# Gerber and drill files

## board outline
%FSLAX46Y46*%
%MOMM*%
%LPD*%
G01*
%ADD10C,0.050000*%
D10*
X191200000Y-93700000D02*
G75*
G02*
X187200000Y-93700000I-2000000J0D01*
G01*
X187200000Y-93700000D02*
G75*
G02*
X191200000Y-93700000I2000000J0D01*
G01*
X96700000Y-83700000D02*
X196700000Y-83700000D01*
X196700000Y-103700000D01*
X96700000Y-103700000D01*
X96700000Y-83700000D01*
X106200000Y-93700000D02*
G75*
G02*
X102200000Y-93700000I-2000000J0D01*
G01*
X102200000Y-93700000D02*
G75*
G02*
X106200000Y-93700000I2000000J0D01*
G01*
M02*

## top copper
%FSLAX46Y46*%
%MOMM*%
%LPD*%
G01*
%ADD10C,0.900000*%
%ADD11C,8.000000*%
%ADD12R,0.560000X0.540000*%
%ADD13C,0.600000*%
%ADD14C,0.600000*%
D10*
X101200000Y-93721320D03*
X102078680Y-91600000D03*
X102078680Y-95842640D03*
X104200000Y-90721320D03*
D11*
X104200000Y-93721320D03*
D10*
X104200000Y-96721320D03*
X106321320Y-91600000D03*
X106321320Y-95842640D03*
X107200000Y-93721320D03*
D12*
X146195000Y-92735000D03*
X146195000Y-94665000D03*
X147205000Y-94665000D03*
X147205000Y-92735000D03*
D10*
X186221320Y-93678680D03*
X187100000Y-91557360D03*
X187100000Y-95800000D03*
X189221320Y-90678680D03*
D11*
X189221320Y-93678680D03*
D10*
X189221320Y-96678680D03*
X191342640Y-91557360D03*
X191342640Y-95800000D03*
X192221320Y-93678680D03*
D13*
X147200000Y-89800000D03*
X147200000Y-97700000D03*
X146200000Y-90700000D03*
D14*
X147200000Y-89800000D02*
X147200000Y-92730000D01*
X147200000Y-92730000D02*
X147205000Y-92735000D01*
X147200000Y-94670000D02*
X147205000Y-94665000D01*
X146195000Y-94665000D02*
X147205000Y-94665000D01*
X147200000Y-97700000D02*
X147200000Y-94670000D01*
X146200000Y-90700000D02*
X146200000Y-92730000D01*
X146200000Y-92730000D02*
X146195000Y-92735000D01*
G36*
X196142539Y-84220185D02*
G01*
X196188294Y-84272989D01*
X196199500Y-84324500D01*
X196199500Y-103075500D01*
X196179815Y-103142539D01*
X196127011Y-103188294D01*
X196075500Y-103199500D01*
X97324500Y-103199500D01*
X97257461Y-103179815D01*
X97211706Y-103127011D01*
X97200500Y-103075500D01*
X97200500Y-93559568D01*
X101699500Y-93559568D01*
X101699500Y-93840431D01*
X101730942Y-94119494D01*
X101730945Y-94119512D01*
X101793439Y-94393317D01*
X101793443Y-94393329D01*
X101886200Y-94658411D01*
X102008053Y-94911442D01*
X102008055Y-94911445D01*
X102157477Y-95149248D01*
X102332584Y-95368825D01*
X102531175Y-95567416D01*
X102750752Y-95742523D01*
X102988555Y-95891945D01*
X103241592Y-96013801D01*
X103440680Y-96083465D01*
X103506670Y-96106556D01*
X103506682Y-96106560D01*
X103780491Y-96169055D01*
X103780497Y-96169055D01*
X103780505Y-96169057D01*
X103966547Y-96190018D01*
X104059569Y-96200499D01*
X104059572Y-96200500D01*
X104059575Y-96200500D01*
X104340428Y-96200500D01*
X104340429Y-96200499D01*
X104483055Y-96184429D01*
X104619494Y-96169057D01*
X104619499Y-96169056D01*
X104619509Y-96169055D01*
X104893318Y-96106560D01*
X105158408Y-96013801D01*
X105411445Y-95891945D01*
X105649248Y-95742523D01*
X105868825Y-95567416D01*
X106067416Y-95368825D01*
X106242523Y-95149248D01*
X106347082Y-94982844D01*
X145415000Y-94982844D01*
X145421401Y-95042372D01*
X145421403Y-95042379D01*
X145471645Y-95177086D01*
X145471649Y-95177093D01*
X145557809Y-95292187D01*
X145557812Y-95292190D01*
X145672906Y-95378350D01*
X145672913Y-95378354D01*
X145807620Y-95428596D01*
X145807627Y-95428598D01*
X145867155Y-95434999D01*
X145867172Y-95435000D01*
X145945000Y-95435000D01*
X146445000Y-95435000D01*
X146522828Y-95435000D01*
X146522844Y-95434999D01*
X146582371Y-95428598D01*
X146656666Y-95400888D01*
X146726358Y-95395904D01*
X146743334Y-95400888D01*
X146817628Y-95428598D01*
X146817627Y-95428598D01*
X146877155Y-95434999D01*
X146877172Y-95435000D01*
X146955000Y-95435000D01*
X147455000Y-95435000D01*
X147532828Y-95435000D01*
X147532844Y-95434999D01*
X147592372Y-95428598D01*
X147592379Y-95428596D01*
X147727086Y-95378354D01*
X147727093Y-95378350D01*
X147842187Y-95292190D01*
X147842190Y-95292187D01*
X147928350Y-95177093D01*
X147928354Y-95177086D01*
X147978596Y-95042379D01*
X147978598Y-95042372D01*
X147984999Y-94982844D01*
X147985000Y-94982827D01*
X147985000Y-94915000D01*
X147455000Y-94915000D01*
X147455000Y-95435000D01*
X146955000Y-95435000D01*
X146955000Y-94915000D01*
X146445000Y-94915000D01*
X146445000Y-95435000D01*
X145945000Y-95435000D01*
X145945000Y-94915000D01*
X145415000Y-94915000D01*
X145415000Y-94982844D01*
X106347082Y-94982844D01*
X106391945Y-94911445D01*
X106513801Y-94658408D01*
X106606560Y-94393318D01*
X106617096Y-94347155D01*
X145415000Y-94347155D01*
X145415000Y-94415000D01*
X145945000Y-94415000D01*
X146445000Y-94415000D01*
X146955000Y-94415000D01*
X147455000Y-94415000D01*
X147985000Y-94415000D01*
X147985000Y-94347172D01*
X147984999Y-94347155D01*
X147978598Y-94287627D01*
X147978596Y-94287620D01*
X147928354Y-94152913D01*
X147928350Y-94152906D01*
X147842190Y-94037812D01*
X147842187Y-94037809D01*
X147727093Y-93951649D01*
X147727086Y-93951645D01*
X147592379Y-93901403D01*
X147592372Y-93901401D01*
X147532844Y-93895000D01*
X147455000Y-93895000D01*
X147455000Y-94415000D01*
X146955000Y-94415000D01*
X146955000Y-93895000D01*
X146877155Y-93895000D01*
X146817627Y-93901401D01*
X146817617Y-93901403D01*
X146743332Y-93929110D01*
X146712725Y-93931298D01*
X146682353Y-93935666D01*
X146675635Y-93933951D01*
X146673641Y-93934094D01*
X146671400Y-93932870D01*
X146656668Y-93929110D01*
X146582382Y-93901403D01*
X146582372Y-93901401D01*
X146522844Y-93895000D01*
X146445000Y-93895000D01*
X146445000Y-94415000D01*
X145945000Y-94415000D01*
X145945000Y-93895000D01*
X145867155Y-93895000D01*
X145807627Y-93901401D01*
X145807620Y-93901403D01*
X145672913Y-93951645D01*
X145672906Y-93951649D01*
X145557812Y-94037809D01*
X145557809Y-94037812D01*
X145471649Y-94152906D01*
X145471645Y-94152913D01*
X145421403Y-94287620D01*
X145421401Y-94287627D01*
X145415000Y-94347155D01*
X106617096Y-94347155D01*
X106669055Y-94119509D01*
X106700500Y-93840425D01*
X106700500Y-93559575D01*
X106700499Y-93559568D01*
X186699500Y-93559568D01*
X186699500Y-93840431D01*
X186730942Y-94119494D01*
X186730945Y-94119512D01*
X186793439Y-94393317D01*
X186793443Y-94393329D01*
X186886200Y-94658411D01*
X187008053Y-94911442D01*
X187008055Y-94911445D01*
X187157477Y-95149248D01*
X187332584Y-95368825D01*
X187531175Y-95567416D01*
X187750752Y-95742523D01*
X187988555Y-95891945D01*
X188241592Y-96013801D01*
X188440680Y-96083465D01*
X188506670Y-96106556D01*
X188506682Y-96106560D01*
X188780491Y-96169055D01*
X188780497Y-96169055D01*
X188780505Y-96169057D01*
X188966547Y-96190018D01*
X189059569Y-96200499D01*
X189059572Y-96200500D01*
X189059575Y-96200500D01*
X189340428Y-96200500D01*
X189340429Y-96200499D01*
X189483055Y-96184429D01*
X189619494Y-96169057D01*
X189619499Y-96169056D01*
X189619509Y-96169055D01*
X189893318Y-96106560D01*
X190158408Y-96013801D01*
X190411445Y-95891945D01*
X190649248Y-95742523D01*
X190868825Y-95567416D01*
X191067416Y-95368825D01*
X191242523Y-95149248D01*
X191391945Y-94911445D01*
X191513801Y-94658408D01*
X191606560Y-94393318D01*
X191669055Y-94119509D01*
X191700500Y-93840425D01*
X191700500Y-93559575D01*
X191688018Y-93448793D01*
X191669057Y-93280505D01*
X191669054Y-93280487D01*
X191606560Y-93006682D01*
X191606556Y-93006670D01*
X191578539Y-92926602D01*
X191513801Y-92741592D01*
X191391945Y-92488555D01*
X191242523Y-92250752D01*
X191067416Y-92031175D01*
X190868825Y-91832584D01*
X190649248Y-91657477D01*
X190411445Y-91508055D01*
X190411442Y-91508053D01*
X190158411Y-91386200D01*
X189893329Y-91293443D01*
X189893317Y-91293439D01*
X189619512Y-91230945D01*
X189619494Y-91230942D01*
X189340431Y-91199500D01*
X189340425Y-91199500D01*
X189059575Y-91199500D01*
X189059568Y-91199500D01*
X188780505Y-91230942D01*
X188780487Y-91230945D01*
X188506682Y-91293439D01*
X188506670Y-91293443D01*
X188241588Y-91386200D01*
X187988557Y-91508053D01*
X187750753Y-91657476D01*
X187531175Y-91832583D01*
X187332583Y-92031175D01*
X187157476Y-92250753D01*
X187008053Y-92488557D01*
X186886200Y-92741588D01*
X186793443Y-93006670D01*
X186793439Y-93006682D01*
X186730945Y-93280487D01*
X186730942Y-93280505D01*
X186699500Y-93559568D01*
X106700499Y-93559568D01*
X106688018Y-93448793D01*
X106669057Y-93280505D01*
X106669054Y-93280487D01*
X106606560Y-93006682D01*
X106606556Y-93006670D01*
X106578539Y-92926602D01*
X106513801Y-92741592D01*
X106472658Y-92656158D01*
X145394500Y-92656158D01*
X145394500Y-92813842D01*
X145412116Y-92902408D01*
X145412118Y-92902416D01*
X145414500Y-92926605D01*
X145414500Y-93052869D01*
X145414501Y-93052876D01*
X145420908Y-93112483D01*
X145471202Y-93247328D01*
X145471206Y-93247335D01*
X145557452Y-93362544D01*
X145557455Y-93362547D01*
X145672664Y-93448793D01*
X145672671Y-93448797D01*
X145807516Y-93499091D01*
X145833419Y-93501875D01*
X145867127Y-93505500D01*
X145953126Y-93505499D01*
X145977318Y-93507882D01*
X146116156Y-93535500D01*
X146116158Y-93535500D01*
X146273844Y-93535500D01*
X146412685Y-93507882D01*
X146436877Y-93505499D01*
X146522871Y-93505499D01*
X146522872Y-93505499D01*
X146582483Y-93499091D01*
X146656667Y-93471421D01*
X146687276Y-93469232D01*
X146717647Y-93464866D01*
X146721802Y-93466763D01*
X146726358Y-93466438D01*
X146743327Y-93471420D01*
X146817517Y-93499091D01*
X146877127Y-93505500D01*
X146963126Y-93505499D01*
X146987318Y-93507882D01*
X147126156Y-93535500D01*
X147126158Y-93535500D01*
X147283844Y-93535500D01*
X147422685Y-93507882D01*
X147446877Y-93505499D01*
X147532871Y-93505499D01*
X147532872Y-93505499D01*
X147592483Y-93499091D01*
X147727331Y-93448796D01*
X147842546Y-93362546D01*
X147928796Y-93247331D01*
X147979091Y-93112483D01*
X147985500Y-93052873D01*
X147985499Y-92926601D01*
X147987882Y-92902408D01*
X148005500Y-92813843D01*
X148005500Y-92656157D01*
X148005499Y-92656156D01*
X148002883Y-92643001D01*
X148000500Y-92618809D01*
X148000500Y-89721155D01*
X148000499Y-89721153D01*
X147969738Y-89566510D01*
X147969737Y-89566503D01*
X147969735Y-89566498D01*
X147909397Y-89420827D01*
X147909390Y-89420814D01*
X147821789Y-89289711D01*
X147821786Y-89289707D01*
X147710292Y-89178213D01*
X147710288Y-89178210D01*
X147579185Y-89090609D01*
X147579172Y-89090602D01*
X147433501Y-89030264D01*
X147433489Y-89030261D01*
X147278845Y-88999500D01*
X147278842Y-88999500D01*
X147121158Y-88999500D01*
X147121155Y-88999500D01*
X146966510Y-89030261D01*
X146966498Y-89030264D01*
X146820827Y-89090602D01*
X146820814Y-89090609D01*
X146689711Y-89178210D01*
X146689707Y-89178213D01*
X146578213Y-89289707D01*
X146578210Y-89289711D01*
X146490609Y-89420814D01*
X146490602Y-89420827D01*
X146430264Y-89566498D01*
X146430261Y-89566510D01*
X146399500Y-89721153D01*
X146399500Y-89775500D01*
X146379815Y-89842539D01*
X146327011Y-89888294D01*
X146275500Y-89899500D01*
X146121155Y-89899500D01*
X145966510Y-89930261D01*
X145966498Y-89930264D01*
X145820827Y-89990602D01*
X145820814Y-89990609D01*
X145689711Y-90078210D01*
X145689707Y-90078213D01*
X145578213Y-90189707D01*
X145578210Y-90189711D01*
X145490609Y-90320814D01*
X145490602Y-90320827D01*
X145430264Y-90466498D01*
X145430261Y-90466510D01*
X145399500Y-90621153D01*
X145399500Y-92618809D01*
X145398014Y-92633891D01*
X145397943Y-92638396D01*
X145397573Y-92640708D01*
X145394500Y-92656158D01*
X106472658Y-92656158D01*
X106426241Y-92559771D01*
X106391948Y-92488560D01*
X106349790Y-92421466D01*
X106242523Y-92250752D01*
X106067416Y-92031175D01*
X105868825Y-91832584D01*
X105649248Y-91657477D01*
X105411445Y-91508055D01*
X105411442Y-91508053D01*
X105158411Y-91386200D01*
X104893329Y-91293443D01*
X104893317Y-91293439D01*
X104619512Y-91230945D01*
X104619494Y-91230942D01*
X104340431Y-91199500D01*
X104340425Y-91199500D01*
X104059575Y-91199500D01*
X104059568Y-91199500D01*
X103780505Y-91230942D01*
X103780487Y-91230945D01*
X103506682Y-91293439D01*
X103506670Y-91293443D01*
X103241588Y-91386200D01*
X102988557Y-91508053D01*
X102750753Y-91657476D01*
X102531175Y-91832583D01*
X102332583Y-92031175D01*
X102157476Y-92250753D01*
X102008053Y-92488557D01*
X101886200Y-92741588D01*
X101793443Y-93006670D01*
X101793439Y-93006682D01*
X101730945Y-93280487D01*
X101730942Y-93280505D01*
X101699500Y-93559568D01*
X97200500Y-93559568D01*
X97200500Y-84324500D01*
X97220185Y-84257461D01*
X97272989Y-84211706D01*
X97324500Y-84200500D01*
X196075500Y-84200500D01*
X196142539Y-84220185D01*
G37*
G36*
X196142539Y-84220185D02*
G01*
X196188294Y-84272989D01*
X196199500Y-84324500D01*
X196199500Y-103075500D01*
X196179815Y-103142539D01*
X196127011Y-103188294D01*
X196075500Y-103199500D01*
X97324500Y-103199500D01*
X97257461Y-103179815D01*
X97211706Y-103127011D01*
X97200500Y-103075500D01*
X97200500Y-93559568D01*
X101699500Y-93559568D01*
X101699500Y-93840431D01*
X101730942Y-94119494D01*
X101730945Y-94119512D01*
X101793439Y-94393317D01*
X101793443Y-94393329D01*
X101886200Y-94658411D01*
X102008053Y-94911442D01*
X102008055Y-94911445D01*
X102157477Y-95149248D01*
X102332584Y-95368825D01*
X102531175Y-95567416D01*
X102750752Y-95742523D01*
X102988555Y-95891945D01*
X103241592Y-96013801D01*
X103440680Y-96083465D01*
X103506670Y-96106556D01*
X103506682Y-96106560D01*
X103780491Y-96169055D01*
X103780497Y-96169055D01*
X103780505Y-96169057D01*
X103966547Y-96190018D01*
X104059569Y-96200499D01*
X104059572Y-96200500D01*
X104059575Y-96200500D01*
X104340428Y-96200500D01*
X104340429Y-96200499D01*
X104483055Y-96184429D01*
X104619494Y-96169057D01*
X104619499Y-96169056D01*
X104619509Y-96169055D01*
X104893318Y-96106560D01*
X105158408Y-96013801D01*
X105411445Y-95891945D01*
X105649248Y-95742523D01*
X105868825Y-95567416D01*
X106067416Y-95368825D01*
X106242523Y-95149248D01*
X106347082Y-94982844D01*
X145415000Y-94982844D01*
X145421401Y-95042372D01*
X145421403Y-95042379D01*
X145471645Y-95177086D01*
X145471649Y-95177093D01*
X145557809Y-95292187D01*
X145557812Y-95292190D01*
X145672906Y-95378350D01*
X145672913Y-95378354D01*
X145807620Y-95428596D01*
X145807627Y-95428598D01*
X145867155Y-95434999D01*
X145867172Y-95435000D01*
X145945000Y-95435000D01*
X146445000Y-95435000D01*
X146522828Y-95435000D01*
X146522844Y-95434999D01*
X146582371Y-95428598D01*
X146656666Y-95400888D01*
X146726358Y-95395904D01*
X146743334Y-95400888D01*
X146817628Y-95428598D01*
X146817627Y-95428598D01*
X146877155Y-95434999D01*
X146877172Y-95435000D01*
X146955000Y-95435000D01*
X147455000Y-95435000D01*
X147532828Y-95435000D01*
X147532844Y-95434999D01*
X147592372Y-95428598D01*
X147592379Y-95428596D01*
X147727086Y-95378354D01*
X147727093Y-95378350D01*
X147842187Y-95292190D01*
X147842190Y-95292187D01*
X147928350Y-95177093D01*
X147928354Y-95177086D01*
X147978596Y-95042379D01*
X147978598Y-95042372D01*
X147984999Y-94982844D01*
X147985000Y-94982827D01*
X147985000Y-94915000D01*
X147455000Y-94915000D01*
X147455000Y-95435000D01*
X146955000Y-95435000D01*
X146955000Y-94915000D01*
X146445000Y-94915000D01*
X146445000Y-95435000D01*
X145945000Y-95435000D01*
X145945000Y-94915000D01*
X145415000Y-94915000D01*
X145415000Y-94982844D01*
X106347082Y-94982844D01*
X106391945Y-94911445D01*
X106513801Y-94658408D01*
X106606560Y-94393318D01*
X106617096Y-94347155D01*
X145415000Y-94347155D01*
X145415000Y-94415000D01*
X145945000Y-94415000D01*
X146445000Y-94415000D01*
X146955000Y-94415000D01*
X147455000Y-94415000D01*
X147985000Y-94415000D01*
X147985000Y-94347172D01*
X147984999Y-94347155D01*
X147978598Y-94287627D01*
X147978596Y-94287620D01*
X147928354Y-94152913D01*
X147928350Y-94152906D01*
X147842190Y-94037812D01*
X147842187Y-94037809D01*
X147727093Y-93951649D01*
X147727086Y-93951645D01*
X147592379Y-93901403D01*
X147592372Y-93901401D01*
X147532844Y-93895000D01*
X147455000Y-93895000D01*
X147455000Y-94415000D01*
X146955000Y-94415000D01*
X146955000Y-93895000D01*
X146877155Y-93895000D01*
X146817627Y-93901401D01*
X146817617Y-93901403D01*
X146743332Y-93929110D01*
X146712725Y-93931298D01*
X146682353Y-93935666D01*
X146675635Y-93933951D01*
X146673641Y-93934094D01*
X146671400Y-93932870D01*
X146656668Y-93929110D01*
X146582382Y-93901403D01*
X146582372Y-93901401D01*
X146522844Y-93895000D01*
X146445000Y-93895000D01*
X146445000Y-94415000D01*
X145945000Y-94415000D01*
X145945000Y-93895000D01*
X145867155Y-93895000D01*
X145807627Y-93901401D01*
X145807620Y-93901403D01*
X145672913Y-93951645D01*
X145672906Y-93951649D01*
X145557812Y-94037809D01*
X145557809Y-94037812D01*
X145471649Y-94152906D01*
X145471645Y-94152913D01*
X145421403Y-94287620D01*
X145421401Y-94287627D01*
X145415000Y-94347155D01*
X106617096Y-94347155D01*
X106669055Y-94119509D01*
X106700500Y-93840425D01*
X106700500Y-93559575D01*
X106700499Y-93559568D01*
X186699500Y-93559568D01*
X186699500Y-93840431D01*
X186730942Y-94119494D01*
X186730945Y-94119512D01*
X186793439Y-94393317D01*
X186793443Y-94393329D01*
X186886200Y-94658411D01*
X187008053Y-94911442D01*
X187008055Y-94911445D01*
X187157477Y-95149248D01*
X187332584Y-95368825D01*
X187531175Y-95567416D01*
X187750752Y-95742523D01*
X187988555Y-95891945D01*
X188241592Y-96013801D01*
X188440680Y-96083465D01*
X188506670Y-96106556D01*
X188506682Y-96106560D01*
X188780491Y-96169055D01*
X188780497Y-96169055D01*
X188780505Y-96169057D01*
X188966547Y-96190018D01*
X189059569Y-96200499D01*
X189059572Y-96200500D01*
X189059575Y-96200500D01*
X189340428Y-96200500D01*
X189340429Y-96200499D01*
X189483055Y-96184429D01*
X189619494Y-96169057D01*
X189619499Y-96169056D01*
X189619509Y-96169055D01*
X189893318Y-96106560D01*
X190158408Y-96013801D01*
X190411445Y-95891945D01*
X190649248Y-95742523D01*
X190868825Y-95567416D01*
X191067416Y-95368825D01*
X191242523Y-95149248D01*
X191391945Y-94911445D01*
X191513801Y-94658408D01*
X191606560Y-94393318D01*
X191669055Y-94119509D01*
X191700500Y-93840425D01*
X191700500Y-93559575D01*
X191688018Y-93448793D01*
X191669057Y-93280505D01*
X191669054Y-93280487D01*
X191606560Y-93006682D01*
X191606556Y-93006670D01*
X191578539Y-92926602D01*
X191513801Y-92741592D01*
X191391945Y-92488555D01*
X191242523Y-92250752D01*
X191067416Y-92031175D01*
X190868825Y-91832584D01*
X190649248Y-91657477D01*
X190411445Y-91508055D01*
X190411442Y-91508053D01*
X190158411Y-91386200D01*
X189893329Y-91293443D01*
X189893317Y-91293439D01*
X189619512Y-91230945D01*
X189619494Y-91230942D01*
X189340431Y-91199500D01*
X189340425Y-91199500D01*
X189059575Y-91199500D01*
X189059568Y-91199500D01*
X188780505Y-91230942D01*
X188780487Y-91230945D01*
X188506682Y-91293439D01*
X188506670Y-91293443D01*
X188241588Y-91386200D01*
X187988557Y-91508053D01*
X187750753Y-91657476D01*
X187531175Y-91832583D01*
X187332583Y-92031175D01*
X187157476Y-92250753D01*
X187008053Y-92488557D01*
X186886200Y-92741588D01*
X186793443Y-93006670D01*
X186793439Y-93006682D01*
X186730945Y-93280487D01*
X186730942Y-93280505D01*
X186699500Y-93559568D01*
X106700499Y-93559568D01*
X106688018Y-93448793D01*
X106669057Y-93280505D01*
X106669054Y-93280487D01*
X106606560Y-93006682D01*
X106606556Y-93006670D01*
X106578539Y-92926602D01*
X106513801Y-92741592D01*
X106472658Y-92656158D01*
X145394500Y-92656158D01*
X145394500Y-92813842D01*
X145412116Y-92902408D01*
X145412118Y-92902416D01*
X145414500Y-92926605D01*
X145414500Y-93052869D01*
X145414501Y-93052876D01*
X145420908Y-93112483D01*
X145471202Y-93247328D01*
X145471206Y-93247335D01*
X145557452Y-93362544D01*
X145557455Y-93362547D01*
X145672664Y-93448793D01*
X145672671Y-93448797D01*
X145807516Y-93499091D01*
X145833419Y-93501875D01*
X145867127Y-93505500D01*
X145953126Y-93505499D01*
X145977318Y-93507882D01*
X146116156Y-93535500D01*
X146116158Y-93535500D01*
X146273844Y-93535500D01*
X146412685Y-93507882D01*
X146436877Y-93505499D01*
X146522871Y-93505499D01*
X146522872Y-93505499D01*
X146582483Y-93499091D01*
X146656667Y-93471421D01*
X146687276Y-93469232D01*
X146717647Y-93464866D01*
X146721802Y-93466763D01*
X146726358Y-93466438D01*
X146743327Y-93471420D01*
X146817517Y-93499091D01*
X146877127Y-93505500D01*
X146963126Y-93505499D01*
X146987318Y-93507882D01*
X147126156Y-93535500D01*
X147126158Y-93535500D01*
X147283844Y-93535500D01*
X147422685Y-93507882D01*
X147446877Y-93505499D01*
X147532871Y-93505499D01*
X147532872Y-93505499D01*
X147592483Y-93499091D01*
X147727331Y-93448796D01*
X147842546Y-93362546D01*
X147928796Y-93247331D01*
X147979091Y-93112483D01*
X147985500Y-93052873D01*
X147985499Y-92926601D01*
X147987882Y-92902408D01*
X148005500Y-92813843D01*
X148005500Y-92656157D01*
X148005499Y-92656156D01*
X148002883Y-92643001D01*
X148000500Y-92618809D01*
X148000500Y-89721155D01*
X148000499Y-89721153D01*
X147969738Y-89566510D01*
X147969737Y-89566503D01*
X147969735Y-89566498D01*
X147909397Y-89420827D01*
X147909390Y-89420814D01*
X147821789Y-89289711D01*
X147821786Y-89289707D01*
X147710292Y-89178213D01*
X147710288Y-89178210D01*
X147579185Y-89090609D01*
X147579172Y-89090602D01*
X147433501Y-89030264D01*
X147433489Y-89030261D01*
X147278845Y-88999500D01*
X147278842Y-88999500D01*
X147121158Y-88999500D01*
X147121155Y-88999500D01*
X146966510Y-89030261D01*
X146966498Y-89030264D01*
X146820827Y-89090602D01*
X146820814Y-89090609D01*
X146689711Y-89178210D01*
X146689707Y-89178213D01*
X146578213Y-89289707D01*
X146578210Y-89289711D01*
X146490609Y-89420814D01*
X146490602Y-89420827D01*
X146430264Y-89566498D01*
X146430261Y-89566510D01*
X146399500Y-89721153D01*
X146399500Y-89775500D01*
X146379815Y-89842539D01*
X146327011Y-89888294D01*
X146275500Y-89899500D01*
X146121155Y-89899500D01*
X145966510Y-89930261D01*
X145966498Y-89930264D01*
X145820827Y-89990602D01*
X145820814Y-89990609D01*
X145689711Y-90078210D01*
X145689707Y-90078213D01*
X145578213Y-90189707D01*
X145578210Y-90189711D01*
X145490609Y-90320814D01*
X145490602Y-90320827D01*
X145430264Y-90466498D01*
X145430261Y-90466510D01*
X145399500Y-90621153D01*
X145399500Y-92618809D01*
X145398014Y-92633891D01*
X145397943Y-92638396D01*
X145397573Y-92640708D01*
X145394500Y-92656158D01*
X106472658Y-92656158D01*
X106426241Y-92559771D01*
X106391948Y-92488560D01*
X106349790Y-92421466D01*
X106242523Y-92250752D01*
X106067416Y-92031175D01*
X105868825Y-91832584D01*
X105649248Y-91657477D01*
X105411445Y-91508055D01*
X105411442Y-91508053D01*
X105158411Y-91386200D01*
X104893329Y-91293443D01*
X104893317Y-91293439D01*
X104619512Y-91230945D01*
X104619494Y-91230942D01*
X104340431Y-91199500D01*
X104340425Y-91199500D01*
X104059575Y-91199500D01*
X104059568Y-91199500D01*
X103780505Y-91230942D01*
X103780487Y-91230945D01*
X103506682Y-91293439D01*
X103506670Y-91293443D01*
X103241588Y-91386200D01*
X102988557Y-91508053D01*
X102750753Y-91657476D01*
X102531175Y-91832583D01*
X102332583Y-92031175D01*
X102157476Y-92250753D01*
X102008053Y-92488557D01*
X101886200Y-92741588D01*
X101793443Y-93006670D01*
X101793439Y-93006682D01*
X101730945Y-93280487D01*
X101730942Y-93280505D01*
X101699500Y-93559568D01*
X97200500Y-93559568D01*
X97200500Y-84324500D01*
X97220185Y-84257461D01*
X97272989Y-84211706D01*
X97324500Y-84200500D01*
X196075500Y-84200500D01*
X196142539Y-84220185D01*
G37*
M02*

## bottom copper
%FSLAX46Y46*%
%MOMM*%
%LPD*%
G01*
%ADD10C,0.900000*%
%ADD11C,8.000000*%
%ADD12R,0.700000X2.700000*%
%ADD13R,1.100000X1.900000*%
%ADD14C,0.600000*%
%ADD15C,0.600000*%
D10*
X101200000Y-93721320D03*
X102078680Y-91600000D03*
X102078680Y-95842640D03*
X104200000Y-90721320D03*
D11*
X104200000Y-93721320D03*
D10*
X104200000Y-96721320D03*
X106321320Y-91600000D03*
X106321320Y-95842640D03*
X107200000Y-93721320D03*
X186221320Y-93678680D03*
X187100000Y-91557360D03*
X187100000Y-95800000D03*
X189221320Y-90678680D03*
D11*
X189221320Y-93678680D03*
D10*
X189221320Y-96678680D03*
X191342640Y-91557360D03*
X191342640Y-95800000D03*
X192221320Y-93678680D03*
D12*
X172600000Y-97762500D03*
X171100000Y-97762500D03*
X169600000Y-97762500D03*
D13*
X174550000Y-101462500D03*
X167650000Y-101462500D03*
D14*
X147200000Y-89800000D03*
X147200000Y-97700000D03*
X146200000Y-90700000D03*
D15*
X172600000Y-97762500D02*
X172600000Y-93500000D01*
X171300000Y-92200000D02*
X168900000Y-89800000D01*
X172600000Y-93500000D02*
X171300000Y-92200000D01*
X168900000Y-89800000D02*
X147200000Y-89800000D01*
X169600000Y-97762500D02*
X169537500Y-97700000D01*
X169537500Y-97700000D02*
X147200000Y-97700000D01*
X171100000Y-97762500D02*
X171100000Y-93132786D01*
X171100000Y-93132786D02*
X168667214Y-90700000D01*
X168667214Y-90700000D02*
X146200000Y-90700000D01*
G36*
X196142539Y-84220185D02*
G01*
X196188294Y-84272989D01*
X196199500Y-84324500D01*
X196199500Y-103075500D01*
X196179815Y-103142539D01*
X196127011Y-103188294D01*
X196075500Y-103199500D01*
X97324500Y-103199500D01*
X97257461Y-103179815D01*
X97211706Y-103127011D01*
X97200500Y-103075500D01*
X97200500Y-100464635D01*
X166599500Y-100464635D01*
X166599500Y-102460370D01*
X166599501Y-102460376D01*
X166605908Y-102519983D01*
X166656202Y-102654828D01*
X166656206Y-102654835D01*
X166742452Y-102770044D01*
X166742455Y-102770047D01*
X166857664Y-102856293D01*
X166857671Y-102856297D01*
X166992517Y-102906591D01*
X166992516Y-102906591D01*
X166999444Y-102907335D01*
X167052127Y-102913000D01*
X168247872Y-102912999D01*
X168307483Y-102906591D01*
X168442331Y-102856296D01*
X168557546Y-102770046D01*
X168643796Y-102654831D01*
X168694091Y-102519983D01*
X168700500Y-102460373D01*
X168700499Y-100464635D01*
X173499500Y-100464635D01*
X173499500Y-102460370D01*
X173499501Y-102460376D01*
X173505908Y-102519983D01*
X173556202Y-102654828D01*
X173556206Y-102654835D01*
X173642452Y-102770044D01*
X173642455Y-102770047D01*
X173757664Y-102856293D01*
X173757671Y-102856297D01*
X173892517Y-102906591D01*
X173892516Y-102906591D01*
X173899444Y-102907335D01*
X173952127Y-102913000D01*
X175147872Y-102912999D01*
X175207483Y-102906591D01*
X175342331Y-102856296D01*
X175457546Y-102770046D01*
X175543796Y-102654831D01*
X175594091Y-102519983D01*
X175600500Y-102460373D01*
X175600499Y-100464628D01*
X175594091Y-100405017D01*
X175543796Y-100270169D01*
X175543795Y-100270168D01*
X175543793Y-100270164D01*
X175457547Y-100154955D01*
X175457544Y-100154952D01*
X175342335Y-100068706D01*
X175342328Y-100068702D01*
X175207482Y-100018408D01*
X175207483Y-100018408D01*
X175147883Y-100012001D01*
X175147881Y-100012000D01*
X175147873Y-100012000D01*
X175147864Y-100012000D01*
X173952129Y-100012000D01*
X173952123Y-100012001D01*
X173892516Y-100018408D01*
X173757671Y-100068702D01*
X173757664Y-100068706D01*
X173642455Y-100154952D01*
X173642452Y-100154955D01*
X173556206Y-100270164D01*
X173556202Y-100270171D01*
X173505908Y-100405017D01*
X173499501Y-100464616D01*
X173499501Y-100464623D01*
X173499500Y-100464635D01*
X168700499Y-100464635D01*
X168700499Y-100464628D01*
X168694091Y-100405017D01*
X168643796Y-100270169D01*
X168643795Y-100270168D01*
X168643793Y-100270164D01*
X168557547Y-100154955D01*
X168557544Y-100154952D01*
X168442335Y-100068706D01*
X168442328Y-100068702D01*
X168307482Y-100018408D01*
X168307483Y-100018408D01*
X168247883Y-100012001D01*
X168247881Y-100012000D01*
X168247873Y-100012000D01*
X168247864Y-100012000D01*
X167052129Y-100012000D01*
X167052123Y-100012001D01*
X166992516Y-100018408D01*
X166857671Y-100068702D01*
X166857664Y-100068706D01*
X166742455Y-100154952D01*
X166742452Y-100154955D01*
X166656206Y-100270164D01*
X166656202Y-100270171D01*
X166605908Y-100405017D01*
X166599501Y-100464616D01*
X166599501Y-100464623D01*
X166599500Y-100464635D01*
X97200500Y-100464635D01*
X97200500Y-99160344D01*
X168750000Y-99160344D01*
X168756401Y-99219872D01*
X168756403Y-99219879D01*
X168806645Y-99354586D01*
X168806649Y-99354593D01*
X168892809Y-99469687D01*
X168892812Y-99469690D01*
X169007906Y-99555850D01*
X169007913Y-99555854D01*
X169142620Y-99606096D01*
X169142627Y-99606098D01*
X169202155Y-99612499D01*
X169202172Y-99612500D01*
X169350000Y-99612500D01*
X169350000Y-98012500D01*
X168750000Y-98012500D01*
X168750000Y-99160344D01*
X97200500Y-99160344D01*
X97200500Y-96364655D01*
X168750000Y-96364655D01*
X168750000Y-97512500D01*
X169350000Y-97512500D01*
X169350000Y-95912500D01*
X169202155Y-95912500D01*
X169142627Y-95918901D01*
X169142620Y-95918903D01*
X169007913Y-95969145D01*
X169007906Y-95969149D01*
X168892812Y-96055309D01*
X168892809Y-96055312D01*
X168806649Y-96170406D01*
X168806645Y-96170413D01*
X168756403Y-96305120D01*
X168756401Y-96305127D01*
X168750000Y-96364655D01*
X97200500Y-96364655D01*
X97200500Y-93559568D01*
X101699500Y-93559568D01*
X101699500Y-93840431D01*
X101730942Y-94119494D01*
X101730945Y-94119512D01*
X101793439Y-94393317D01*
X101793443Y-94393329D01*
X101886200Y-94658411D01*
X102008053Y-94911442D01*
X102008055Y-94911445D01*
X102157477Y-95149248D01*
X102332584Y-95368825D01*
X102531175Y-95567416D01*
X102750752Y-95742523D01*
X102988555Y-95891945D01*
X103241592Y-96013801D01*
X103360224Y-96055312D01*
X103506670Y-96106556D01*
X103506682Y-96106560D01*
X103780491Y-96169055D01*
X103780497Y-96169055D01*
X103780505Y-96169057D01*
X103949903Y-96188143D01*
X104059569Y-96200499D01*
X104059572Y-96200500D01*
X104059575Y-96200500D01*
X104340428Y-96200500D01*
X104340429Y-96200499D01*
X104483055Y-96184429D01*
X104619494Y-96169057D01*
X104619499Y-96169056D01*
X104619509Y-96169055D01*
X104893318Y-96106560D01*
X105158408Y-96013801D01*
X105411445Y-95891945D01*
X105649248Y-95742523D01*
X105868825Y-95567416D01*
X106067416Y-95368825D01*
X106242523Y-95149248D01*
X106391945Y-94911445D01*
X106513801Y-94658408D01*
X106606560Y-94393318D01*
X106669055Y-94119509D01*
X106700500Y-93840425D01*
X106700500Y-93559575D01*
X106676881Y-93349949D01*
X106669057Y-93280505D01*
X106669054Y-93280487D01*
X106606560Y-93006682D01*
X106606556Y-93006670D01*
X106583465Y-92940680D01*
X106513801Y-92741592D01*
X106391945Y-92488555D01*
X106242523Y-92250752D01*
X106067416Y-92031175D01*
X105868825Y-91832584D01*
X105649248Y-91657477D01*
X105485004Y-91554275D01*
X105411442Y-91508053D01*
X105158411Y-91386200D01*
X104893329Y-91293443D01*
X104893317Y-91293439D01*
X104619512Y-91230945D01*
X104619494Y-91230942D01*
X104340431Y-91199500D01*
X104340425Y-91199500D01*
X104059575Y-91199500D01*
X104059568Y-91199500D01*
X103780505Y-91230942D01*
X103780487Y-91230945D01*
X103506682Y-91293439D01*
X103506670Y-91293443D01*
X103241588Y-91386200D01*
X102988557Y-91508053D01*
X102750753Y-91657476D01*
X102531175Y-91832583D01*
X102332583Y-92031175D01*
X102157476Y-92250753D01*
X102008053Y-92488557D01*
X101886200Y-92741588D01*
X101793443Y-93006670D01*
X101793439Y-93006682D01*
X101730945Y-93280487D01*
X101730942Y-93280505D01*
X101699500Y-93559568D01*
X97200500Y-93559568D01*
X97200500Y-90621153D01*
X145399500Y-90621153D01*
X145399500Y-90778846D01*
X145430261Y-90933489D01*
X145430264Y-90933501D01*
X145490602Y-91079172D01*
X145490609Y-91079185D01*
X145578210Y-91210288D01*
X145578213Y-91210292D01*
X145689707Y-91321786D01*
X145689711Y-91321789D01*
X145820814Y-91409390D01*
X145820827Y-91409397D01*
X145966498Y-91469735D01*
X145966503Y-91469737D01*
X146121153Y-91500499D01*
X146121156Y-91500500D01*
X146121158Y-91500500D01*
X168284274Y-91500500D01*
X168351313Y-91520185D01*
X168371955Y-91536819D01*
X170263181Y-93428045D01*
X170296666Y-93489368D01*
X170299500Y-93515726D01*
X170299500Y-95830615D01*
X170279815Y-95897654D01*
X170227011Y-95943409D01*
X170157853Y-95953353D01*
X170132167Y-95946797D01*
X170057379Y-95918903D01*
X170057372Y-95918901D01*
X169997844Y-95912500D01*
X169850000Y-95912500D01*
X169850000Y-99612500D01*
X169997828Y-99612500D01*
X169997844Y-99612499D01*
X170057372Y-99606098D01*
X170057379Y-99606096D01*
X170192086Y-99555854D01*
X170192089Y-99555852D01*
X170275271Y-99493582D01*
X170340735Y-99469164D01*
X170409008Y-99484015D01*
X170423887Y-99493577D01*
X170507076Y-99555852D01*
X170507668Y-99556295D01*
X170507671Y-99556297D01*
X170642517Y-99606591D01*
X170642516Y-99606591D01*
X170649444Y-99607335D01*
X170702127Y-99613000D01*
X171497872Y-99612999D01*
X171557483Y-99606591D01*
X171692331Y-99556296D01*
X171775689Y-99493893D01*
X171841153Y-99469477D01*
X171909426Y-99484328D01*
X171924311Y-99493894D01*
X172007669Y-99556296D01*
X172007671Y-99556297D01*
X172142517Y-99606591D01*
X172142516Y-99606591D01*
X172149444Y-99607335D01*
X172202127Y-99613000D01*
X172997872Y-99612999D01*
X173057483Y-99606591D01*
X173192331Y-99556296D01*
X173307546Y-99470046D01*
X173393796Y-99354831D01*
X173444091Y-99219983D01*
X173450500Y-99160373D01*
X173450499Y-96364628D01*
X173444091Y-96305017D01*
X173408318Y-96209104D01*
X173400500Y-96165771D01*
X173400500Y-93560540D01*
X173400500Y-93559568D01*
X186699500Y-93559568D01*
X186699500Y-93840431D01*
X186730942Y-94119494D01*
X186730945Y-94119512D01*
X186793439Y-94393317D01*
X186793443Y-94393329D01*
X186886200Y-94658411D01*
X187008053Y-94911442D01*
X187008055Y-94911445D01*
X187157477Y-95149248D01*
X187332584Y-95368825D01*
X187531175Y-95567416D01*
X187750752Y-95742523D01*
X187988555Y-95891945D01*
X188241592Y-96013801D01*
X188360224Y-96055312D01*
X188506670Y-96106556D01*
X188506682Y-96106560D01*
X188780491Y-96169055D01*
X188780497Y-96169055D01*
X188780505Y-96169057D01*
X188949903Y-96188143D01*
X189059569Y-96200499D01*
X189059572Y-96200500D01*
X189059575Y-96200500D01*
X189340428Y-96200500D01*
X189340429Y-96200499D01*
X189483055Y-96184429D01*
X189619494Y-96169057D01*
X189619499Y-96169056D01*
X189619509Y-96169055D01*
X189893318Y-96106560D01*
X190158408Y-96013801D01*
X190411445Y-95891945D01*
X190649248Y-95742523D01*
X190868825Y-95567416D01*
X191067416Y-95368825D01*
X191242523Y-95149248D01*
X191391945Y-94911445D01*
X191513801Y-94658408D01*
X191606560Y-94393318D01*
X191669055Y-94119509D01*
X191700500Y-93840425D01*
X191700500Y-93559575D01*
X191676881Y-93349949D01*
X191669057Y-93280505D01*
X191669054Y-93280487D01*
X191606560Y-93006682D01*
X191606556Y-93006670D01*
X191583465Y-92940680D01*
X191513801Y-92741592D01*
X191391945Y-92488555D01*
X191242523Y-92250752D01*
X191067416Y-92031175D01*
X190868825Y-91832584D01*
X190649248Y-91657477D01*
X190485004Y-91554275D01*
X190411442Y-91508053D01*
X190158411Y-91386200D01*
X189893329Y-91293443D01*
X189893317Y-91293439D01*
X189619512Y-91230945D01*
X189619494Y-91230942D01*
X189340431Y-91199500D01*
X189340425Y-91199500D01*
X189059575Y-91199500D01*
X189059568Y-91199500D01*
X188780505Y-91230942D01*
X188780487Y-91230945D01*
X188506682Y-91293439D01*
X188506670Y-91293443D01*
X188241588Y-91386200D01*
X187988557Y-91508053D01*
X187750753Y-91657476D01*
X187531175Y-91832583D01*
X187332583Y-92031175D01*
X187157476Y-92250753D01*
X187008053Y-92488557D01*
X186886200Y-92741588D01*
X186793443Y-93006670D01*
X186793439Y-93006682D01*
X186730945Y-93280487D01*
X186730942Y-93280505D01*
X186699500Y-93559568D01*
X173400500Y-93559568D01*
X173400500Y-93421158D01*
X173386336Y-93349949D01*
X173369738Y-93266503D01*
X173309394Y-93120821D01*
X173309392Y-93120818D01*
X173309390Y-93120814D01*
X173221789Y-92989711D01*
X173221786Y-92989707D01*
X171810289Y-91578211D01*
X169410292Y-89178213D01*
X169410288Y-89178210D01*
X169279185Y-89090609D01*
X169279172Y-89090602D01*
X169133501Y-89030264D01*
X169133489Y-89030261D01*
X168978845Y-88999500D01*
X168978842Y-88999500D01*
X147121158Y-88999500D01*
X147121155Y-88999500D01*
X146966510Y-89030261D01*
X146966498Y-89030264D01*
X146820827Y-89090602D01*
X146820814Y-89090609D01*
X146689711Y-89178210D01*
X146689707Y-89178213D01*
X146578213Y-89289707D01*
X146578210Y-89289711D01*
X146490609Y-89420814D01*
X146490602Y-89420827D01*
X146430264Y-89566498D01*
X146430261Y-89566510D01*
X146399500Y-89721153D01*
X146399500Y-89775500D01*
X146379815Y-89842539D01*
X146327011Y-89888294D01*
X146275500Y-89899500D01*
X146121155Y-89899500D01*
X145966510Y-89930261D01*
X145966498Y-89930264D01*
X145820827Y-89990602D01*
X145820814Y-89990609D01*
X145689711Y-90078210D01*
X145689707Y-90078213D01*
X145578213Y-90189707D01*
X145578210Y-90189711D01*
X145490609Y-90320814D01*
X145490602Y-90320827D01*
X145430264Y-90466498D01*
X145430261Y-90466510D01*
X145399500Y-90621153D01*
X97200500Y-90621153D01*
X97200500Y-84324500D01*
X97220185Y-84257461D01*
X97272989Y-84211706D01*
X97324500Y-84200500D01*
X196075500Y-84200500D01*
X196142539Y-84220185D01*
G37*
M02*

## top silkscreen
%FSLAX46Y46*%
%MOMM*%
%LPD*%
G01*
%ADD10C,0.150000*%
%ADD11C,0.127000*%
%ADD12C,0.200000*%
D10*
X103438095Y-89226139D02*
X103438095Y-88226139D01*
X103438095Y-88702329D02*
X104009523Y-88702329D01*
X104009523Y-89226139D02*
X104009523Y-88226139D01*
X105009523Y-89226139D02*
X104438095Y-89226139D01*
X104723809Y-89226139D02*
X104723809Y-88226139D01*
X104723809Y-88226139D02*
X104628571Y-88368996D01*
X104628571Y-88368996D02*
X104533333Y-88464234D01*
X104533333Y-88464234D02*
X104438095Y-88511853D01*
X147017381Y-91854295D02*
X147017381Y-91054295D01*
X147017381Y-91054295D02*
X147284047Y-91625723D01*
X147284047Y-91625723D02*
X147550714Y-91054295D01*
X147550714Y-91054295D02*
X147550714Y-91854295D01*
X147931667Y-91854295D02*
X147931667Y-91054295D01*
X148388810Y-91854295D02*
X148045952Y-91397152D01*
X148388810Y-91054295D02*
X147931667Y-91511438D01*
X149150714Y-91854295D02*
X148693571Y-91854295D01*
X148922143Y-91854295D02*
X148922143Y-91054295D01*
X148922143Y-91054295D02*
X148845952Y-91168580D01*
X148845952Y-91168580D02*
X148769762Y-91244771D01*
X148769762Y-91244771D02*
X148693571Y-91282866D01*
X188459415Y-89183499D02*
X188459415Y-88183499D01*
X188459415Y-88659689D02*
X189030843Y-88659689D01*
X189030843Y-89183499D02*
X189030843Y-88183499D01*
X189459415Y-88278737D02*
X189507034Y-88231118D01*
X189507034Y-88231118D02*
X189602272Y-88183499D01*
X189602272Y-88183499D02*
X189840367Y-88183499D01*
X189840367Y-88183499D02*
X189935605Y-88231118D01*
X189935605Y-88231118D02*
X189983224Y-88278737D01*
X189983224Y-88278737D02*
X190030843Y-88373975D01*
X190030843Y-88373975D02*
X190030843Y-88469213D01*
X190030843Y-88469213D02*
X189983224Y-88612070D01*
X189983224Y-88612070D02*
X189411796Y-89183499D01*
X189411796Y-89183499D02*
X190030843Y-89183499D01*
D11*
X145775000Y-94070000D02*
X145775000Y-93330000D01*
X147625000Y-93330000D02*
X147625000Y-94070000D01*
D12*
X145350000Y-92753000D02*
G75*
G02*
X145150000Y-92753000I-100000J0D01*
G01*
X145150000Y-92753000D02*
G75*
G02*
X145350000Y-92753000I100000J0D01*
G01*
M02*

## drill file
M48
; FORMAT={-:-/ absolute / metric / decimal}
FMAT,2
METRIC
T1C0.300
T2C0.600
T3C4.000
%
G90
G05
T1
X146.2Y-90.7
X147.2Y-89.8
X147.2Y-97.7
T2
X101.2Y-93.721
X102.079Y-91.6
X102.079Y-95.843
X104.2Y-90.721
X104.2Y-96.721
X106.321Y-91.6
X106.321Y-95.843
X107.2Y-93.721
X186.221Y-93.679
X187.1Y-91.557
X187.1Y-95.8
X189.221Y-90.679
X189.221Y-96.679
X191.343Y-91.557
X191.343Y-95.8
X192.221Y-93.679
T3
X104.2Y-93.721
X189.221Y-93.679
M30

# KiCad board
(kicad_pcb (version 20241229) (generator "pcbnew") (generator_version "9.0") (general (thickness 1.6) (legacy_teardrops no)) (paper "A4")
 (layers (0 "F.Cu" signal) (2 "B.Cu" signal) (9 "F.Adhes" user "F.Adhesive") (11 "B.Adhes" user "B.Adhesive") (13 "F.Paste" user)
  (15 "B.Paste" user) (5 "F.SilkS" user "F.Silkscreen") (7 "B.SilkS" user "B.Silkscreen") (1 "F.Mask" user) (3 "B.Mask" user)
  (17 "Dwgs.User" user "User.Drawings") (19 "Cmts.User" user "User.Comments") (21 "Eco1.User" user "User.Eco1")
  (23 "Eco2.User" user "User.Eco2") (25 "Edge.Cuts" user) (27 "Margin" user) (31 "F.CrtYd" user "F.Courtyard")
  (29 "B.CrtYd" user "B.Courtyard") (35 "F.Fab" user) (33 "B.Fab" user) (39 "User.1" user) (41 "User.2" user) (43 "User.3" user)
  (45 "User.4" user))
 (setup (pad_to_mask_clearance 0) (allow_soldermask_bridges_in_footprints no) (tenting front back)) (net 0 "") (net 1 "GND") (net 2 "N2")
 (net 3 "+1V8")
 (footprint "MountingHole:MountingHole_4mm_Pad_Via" (layer "F.Cu") (at 104.2 93.72132)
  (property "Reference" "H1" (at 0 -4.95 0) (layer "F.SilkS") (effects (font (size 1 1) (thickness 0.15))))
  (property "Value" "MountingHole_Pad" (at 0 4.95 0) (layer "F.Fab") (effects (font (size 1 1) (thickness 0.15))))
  (pad "1" thru_hole circle (at -3 0) (size 0.9 0.9) (drill 0.6) (layers "*.Cu" "*.Mask") (remove_unused_layers no) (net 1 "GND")
   (zone_connect 2))
  (pad "1" thru_hole circle (at -2.12132 -2.12132) (size 0.9 0.9) (drill 0.6) (layers "*.Cu" "*.Mask") (remove_unused_layers no)
   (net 1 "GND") (zone_connect 2))
  (pad "1" thru_hole circle (at -2.12132 2.12132) (size 0.9 0.9) (drill 0.6) (layers "*.Cu" "*.Mask") (remove_unused_layers no)
   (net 1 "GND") (zone_connect 2))
  (pad "1" thru_hole circle (at 0 -3) (size 0.9 0.9) (drill 0.6) (layers "*.Cu" "*.Mask") (remove_unused_layers no) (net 1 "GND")
   (zone_connect 2))
  (pad "1" thru_hole circle (at 0 0) (size 8 8) (drill 4) (layers "*.Cu" "*.Mask") (remove_unused_layers no) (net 1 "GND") (zone_connect 2))
  (pad "1" thru_hole circle (at 0 3) (size 0.9 0.9) (drill 0.6) (layers "*.Cu" "*.Mask") (remove_unused_layers no) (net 1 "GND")
   (zone_connect 2))
  (pad "1" thru_hole circle (at 2.12132 -2.12132) (size 0.9 0.9) (drill 0.6) (layers "*.Cu" "*.Mask") (remove_unused_layers no)
   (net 1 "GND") (zone_connect 2))
  (pad "1" thru_hole circle (at 2.12132 2.12132) (size 0.9 0.9) (drill 0.6) (layers "*.Cu" "*.Mask") (remove_unused_layers no) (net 1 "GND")
   (zone_connect 2))
  (pad "1" thru_hole circle (at 3 0) (size 0.9 0.9) (drill 0.6) (layers "*.Cu" "*.Mask") (remove_unused_layers no) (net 1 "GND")
   (zone_connect 2)))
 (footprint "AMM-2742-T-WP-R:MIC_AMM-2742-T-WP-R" (layer "F.Cu") (at 146.7 93.7)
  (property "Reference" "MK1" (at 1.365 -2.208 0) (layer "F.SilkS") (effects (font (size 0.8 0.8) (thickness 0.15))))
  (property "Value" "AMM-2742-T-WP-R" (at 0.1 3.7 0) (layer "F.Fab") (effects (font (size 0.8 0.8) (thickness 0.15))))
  (fp_line (start -0.925 0.37) (end -0.925 -0.37) (stroke (width 0.127) (type solid)) (layer "F.SilkS"))
  (fp_line (start 0.925 -0.37) (end 0.925 0.37) (stroke (width 0.127) (type solid)) (layer "F.SilkS"))
  (fp_circle (center -1.45 -0.947) (end -1.35 -0.947) (stroke (width 0.2) (type solid)) (fill no) (layer "F.SilkS"))
  (pad "1" smd rect (at -0.505 -0.965) (size 0.56 0.54) (layers "F.Cu" "F.Mask" "F.Paste") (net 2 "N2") (solder_mask_margin 0.102))
  (pad "2" smd rect (at -0.505 0.965) (size 0.56 0.54) (layers "F.Cu" "F.Mask" "F.Paste") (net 1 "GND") (solder_mask_margin 0.102))
  (pad "3" smd rect (at 0.505 0.965) (size 0.56 0.54) (layers "F.Cu" "F.Mask" "F.Paste") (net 1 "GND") (solder_mask_margin 0.102))
  (pad "4" smd rect (at 0.505 -0.965) (size 0.56 0.54) (layers "F.Cu" "F.Mask" "F.Paste") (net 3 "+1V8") (solder_mask_margin 0.102)))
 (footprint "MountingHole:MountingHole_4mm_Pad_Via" (layer "F.Cu") (at 189.22132 93.67868)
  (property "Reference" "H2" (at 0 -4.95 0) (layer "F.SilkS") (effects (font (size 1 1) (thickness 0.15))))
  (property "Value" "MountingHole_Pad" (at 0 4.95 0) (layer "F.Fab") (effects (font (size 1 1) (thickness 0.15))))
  (pad "1" thru_hole circle (at -3 0) (size 0.9 0.9) (drill 0.6) (layers "*.Cu" "*.Mask") (remove_unused_layers no) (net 1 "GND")
   (zone_connect 2))
  (pad "1" thru_hole circle (at -2.12132 -2.12132) (size 0.9 0.9) (drill 0.6) (layers "*.Cu" "*.Mask") (remove_unused_layers no)
   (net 1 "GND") (zone_connect 2))
  (pad "1" thru_hole circle (at -2.12132 2.12132) (size 0.9 0.9) (drill 0.6) (layers "*.Cu" "*.Mask") (remove_unused_layers no)
   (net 1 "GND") (zone_connect 2))
  (pad "1" thru_hole circle (at 0 -3) (size 0.9 0.9) (drill 0.6) (layers "*.Cu" "*.Mask") (remove_unused_layers no) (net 1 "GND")
   (zone_connect 2))
  (pad "1" thru_hole circle (at 0 0) (size 8 8) (drill 4) (layers "*.Cu" "*.Mask") (remove_unused_layers no) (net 1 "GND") (zone_connect 2))
  (pad "1" thru_hole circle (at 0 3) (size 0.9 0.9) (drill 0.6) (layers "*.Cu" "*.Mask") (remove_unused_layers no) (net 1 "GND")
   (zone_connect 2))
  (pad "1" thru_hole circle (at 2.12132 -2.12132) (size 0.9 0.9) (drill 0.6) (layers "*.Cu" "*.Mask") (remove_unused_layers no)
   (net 1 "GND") (zone_connect 2))
  (pad "1" thru_hole circle (at 2.12132 2.12132) (size 0.9 0.9) (drill 0.6) (layers "*.Cu" "*.Mask") (remove_unused_layers no) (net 1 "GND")
   (zone_connect 2))
  (pad "1" thru_hole circle (at 3 0) (size 0.9 0.9) (drill 0.6) (layers "*.Cu" "*.Mask") (remove_unused_layers no) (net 1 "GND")
   (zone_connect 2)))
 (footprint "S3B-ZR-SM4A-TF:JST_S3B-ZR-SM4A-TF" (layer "B.Cu") (at 171.1 101.4625 180)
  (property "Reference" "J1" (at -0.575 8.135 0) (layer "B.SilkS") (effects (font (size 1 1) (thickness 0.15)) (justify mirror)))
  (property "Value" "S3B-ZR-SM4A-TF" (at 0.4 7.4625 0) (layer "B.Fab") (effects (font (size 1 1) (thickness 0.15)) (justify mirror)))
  (pad "1" smd rect (at -1.5 3.7 180) (size 0.7 2.7) (layers "B.Cu" "B.Mask" "B.Paste") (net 3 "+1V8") (solder_mask_margin 0.102))
  (pad "2" smd rect (at 0 3.7 180) (size 0.7 2.7) (layers "B.Cu" "B.Mask" "B.Paste") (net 2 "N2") (solder_mask_margin 0.102))
  (pad "3" smd rect (at 1.5 3.7 180) (size 0.7 2.7) (layers "B.Cu" "B.Mask" "B.Paste") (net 1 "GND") (solder_mask_margin 0.102))
  (pad "SH1" smd rect (at -3.45 0 180) (size 1.1 1.9) (layers "B.Cu" "B.Mask" "B.Paste") (solder_mask_margin 0.102))
  (pad "SH2" smd rect (at 3.45 0 180) (size 1.1 1.9) (layers "B.Cu" "B.Mask" "B.Paste") (solder_mask_margin 0.102)))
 (gr_circle (center 189.2 93.7) (end 191.2 93.7) (stroke (width 0.05) (type solid)) (fill no) (layer "Edge.Cuts"))
 (gr_rect (start 96.7 83.7) (end 196.7 103.7) (stroke (width 0.05) (type solid)) (fill no) (layer "Edge.Cuts"))
 (gr_circle (center 104.2 93.7) (end 106.2 93.7) (stroke (width 0.05) (type solid)) (fill no) (layer "Edge.Cuts"))
 (segment (start 147.2 89.8) (end 147.2 92.73) (width 0.6) (layer "F.Cu") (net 3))
 (segment (start 147.2 92.73) (end 147.205 92.735) (width 0.6) (layer "F.Cu") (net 3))
 (via (at 147.2 89.8) (size 0.6) (drill 0.3) (layers "F.Cu" "B.Cu") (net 3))
 (segment (start 172.6 97.7625) (end 172.6 93.5) (width 0.6) (layer "B.Cu") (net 3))
 (segment (start 171.3 92.2) (end 168.9 89.8) (width 0.6) (layer "B.Cu") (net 3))
 (segment (start 172.6 93.5) (end 171.3 92.2) (width 0.6) (layer "B.Cu") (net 3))
 (segment (start 168.9 89.8) (end 147.2 89.8) (width 0.6) (layer "B.Cu") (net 3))
 (segment (start 147.2 94.67) (end 147.205 94.665) (width 0.6) (layer "F.Cu") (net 1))
 (segment (start 146.195 94.665) (end 147.205 94.665) (width 0.6) (layer "F.Cu") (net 1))
 (segment (start 147.2 97.7) (end 147.2 94.67) (width 0.6) (layer "F.Cu") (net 1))
 (via (at 147.2 97.7) (size 0.6) (drill 0.3) (layers "F.Cu" "B.Cu") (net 1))
 (segment (start 169.6 97.7625) (end 169.5375 97.7) (width 0.6) (layer "B.Cu") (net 1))
 (segment (start 169.5375 97.7) (end 147.2 97.7) (width 0.6) (layer "B.Cu") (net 1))
 (segment (start 146.2 90.7) (end 146.2 92.73) (width 0.6) (layer "F.Cu") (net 2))
 (segment (start 146.2 92.73) (end 146.195 92.735) (width 0.6) (layer "F.Cu") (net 2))
 (via (at 146.2 90.7) (size 0.6) (drill 0.3) (layers "F.Cu" "B.Cu") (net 2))
 (segment (start 171.1 97.7625) (end 171.1 93.132786) (width 0.6) (layer "B.Cu") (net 2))
 (segment (start 171.1 93.132786) (end 168.667214 90.7) (width 0.6) (layer "B.Cu") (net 2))
 (segment (start 168.667214 90.7) (end 146.2 90.7) (width 0.6) (layer "B.Cu") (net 2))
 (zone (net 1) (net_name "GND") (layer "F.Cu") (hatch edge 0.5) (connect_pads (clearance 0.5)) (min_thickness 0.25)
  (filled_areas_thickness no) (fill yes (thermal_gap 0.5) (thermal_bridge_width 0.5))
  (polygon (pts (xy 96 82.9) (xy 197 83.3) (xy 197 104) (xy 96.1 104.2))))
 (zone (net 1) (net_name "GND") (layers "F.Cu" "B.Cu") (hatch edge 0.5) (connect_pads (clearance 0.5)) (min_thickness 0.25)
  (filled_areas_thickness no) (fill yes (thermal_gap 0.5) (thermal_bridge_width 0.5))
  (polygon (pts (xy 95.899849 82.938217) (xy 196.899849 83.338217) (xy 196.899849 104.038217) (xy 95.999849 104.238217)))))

